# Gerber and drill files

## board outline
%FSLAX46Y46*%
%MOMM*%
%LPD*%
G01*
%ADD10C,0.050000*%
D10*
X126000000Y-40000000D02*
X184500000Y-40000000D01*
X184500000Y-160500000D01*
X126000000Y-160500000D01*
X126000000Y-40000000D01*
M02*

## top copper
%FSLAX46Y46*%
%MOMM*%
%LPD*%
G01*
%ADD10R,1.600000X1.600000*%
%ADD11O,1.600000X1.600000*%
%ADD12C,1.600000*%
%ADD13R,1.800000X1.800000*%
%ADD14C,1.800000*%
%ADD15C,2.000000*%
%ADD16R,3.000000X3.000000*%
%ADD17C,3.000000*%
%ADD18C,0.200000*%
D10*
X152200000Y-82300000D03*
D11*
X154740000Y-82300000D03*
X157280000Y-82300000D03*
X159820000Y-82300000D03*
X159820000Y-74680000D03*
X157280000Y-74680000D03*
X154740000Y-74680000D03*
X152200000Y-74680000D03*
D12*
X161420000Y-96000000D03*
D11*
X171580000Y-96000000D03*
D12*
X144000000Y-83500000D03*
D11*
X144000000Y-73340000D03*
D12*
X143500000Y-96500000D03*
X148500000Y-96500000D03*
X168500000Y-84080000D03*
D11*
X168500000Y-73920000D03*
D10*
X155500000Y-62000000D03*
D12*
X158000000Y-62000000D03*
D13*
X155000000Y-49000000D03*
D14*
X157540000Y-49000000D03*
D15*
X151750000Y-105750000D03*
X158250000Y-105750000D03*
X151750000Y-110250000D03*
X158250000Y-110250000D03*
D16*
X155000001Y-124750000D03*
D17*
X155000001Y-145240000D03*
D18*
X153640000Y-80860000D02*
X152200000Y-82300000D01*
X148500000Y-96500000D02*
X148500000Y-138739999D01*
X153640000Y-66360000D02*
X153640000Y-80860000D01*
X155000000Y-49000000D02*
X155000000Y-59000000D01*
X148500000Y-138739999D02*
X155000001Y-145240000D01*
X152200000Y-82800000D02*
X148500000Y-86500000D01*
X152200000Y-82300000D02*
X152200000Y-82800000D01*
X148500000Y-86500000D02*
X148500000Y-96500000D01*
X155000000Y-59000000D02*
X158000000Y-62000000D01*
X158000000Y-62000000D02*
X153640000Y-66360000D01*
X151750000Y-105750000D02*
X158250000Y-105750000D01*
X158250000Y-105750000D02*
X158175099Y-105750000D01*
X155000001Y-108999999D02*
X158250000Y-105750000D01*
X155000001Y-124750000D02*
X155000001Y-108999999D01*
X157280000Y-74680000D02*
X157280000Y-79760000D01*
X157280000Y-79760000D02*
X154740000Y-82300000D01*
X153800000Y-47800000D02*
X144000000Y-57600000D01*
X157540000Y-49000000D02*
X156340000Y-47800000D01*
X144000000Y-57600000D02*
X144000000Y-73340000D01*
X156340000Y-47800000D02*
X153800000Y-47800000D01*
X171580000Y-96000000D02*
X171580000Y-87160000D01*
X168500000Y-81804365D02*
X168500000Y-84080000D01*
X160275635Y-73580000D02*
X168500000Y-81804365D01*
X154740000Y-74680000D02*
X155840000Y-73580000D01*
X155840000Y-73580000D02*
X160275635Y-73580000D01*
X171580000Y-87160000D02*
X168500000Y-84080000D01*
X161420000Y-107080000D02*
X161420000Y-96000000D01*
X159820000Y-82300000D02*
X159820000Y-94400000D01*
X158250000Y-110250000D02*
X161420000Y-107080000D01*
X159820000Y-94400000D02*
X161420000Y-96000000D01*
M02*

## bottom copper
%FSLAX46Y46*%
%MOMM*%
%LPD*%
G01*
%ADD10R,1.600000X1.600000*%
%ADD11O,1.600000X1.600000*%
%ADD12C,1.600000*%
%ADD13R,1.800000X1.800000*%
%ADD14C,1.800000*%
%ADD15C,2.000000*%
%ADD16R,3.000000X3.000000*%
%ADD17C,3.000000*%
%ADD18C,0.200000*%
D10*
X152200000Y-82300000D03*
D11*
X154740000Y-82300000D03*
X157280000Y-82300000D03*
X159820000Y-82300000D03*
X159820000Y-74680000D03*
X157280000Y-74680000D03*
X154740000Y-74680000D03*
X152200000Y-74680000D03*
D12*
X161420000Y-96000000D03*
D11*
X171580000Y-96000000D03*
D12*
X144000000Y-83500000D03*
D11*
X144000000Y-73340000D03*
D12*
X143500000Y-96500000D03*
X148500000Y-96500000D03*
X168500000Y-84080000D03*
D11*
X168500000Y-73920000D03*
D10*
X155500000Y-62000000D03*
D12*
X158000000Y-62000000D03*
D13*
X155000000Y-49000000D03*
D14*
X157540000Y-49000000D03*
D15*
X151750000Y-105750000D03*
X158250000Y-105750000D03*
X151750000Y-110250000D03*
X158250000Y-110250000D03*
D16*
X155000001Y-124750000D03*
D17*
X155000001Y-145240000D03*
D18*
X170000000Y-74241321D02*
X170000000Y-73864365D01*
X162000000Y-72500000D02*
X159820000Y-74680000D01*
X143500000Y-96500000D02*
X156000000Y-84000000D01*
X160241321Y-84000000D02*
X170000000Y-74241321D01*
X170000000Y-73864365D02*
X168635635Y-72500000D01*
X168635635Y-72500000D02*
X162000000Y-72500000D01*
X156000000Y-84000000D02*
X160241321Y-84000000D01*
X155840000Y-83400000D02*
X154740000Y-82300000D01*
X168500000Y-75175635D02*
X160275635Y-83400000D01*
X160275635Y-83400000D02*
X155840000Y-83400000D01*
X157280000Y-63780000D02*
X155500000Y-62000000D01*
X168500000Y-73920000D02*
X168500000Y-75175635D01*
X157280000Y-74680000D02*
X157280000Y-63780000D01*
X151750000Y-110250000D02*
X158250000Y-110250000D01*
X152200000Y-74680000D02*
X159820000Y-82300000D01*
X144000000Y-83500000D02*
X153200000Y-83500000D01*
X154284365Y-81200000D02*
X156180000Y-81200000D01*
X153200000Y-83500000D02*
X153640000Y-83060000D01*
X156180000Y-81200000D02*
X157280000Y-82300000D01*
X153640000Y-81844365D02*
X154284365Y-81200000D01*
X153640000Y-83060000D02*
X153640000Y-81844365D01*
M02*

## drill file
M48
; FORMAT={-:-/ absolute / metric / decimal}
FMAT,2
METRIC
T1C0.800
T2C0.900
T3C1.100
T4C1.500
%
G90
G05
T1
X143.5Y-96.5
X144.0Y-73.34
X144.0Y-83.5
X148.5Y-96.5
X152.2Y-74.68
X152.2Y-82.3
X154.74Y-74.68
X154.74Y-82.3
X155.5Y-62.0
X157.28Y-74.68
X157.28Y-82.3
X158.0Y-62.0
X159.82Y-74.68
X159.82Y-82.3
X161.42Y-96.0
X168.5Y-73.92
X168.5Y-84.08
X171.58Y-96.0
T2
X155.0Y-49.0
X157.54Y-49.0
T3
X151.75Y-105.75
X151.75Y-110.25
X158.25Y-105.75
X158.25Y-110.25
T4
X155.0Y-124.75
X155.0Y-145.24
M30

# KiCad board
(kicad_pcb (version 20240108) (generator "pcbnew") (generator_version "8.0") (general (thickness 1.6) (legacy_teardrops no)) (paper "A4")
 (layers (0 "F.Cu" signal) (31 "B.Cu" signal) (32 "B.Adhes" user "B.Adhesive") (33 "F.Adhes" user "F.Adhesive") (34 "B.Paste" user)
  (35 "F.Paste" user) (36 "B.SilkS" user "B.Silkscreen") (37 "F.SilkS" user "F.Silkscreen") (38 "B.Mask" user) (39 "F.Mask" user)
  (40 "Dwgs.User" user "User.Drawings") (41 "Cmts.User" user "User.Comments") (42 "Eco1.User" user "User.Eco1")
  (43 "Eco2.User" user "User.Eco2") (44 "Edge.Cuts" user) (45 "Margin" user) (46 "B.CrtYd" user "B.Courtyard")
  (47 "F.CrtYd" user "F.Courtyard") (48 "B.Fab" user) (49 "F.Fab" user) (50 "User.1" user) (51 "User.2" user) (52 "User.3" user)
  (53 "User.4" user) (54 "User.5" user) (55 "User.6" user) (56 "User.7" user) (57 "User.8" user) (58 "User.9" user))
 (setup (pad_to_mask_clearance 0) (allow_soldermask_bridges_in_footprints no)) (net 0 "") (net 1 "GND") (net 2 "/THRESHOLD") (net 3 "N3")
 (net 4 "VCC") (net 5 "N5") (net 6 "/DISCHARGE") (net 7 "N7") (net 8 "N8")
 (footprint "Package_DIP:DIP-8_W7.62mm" (layer "F.Cu") (at 152.2 82.3 90)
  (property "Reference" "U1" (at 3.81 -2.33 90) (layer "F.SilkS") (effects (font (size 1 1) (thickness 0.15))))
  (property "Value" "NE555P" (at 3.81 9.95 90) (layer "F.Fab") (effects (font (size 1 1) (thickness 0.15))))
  (pad "1" thru_hole rect (at 0 0 90) (size 1.6 1.6) (drill 0.8) (layers "*.Cu" "*.Mask") (remove_unused_layers no) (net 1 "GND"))
  (pad "2" thru_hole oval (at 0 2.54 90) (size 1.6 1.6) (drill 0.8) (layers "*.Cu" "*.Mask") (remove_unused_layers no) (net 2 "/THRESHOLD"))
  (pad "3" thru_hole oval (at 0 5.08 90) (size 1.6 1.6) (drill 0.8) (layers "*.Cu" "*.Mask") (remove_unused_layers no) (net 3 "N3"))
  (pad "4" thru_hole oval (at 0 7.62 90) (size 1.6 1.6) (drill 0.8) (layers "*.Cu" "*.Mask") (remove_unused_layers no) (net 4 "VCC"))
  (pad "5" thru_hole oval (at 7.62 7.62 90) (size 1.6 1.6) (drill 0.8) (layers "*.Cu" "*.Mask") (remove_unused_layers no) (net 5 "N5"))
  (pad "6" thru_hole oval (at 7.62 5.08 90) (size 1.6 1.6) (drill 0.8) (layers "*.Cu" "*.Mask") (remove_unused_layers no)
   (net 2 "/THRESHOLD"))
  (pad "7" thru_hole oval (at 7.62 2.54 90) (size 1.6 1.6) (drill 0.8) (layers "*.Cu" "*.Mask") (remove_unused_layers no)
   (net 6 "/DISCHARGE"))
  (pad "8" thru_hole oval (at 7.62 0 90) (size 1.6 1.6) (drill 0.8) (layers "*.Cu" "*.Mask") (remove_unused_layers no) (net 4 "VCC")))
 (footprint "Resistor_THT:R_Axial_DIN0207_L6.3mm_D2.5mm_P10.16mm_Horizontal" (layer "F.Cu") (at 161.42 96)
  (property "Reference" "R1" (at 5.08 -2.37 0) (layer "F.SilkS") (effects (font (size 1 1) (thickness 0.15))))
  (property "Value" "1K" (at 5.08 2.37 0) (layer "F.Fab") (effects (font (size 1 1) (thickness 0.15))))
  (pad "1" thru_hole circle (at 0 0) (size 1.6 1.6) (drill 0.8) (layers "*.Cu" "*.Mask") (remove_unused_layers no) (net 4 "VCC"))
  (pad "2" thru_hole oval (at 10.16 0) (size 1.6 1.6) (drill 0.8) (layers "*.Cu" "*.Mask") (remove_unused_layers no) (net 6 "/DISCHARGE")))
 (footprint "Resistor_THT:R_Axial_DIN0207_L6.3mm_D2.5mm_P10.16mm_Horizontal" (layer "F.Cu") (at 144 83.5 90)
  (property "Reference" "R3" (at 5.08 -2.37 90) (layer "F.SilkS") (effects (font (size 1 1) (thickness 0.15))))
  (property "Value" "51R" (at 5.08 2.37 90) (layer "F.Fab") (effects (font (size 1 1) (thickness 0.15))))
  (pad "1" thru_hole circle (at 0 0 90) (size 1.6 1.6) (drill 0.8) (layers "*.Cu" "*.Mask") (remove_unused_layers no) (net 3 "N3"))
  (pad "2" thru_hole oval (at 10.16 0 90) (size 1.6 1.6) (drill 0.8) (layers "*.Cu" "*.Mask") (remove_unused_layers no) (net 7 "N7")))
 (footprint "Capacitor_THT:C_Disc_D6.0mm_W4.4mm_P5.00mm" (layer "F.Cu") (at 143.5 96.5)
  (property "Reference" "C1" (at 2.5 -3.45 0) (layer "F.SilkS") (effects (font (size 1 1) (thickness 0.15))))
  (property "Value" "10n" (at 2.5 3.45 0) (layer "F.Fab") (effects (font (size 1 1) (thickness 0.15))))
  (pad "1" thru_hole circle (at 0 0) (size 1.6 1.6) (drill 0.8) (layers "*.Cu" "*.Mask") (remove_unused_layers no) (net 5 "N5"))
  (pad "2" thru_hole circle (at 5 0) (size 1.6 1.6) (drill 0.8) (layers "*.Cu" "*.Mask") (remove_unused_layers no) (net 1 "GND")))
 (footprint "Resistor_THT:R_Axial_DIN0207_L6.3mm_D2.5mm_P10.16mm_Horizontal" (layer "F.Cu") (at 168.5 84.08 90)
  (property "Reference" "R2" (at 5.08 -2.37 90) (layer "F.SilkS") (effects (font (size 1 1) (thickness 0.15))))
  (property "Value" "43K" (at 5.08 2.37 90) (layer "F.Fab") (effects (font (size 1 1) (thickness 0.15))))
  (pad "1" thru_hole circle (at 0 0 90) (size 1.6 1.6) (drill 0.8) (layers "*.Cu" "*.Mask") (remove_unused_layers no) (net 6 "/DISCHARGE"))
  (pad "2" thru_hole oval (at 10.16 0 90) (size 1.6 1.6) (drill 0.8) (layers "*.Cu" "*.Mask") (remove_unused_layers no) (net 2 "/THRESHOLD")))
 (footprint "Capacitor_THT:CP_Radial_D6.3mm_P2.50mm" (layer "F.Cu") (at 155.5 62)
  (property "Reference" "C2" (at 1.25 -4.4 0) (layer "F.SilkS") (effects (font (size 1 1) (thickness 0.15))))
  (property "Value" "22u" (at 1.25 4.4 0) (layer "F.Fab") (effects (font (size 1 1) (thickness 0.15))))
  (pad "1" thru_hole rect (at 0 0) (size 1.6 1.6) (drill 0.8) (layers "*.Cu" "*.Mask") (remove_unused_layers no) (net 2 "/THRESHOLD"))
  (pad "2" thru_hole circle (at 2.5 0) (size 1.6 1.6) (drill 0.8) (layers "*.Cu" "*.Mask") (remove_unused_layers no) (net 1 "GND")))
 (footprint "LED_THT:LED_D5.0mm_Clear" (layer "F.Cu") (at 155 49)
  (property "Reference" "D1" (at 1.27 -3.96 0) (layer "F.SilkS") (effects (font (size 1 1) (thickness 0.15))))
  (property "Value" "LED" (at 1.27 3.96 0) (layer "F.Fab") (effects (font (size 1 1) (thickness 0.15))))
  (pad "1" thru_hole rect (at 0 0) (size 1.8 1.8) (drill 0.9) (layers "*.Cu" "*.Mask") (remove_unused_layers no) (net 1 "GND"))
  (pad "2" thru_hole circle (at 2.54 0) (size 1.8 1.8) (drill 0.9) (layers "*.Cu" "*.Mask") (remove_unused_layers no) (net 7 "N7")))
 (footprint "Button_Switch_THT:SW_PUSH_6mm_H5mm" (layer "F.Cu") (at 151.75 105.75)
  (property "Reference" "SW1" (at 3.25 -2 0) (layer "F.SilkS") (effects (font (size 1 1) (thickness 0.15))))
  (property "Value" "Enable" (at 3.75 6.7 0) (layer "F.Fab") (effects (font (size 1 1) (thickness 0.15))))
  (pad "1" thru_hole circle (at 0 0 90) (size 2 2) (drill 1.1) (layers "*.Cu" "*.Mask") (remove_unused_layers no) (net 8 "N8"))
  (pad "1" thru_hole circle (at 6.5 0 90) (size 2 2) (drill 1.1) (layers "*.Cu" "*.Mask") (remove_unused_layers no) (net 8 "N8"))
  (pad "2" thru_hole circle (at 0 4.5 90) (size 2 2) (drill 1.1) (layers "*.Cu" "*.Mask") (remove_unused_layers no) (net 4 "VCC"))
  (pad "2" thru_hole circle (at 6.5 4.5 90) (size 2 2) (drill 1.1) (layers "*.Cu" "*.Mask") (remove_unused_layers no) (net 4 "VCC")))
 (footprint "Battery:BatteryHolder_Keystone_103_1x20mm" (layer "F.Cu") (at 155.000001 124.75 -90)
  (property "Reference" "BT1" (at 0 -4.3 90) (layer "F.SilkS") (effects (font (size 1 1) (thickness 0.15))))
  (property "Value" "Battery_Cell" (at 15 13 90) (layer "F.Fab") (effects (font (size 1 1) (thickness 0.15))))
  (pad "1" thru_hole rect (at 0 0 270) (size 3 3) (drill 1.5) (layers "*.Cu" "*.Mask") (remove_unused_layers no) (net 8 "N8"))
  (pad "2" thru_hole circle (at 20.49 0 270) (size 3 3) (drill 1.5) (layers "*.Cu" "*.Mask") (remove_unused_layers no) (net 1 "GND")))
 (gr_rect (start 126 40) (end 184.5 160.5) (stroke (width 0.05) (type default)) (fill none) (layer "Edge.Cuts"))
 (segment (start 153.64 80.86) (end 152.2 82.3) (width 0.2) (layer "F.Cu") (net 1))
 (segment (start 148.5 96.5) (end 148.5 138.739999) (width 0.2) (layer "F.Cu") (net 1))
 (segment (start 153.64 66.36) (end 153.64 80.86) (width 0.2) (layer "F.Cu") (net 1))
 (segment (start 155 49) (end 155 59) (width 0.2) (layer "F.Cu") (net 1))
 (segment (start 148.5 138.739999) (end 155.000001 145.24) (width 0.2) (layer "F.Cu") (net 1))
 (segment (start 152.2 82.8) (end 148.5 86.5) (width 0.2) (layer "F.Cu") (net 1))
 (segment (start 152.2 82.3) (end 152.2 82.8) (width 0.2) (layer "F.Cu") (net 1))
 (segment (start 148.5 86.5) (end 148.5 96.5) (width 0.2) (layer "F.Cu") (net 1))
 (segment (start 155 59) (end 158 62) (width 0.2) (layer "F.Cu") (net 1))
 (segment (start 158 62) (end 153.64 66.36) (width 0.2) (layer "F.Cu") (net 1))
 (segment (start 151.75 105.75) (end 158.25 105.75) (width 0.2) (layer "F.Cu") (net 8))
 (segment (start 158.25 105.75) (end 158.175099 105.75) (width 0.2) (layer "F.Cu") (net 8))
 (segment (start 155.000001 108.999999) (end 158.25 105.75) (width 0.2) (layer "F.Cu") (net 8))
 (segment (start 155.000001 124.75) (end 155.000001 108.999999) (width 0.2) (layer "F.Cu") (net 8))
 (segment (start 170 74.241321) (end 170 73.864365) (width 0.2) (layer "B.Cu") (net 5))
 (segment (start 162 72.5) (end 159.82 74.68) (width 0.2) (layer "B.Cu") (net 5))
 (segment (start 143.5 96.5) (end 156 84) (width 0.2) (layer "B.Cu") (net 5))
 (segment (start 160.241321 84) (end 170 74.241321) (width 0.2) (layer "B.Cu") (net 5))
 (segment (start 170 73.864365) (end 168.635635 72.5) (width 0.2) (layer "B.Cu") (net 5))
 (segment (start 168.635635 72.5) (end 162 72.5) (width 0.2) (layer "B.Cu") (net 5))
 (segment (start 156 84) (end 160.241321 84) (width 0.2) (layer "B.Cu") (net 5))
 (segment (start 157.28 74.68) (end 157.28 79.76) (width 0.2) (layer "F.Cu") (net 2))
 (segment (start 157.28 79.76) (end 154.74 82.3) (width 0.2) (layer "F.Cu") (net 2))
 (segment (start 155.84 83.4) (end 154.74 82.3) (width 0.2) (layer "B.Cu") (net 2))
 (segment (start 168.5 75.175635) (end 160.275635 83.4) (width 0.2) (layer "B.Cu") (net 2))
 (segment (start 160.275635 83.4) (end 155.84 83.4) (width 0.2) (layer "B.Cu") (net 2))
 (segment (start 157.28 63.78) (end 155.5 62) (width 0.2) (layer "B.Cu") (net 2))
 (segment (start 168.5 73.92) (end 168.5 75.175635) (width 0.2) (layer "B.Cu") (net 2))
 (segment (start 157.28 74.68) (end 157.28 63.78) (width 0.2) (layer "B.Cu") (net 2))
 (segment (start 153.8 47.8) (end 144 57.6) (width 0.2) (layer "F.Cu") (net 7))
 (segment (start 157.54 49) (end 156.34 47.8) (width 0.2) (layer "F.Cu") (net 7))
 (segment (start 144 57.6) (end 144 73.34) (width 0.2) (layer "F.Cu") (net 7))
 (segment (start 156.34 47.8) (end 153.8 47.8) (width 0.2) (layer "F.Cu") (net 7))
 (segment (start 171.58 96) (end 171.58 87.16) (width 0.2) (layer "F.Cu") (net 6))
 (segment (start 168.5 81.804365) (end 168.5 84.08) (width 0.2) (layer "F.Cu") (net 6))
 (segment (start 160.275635 73.58) (end 168.5 81.804365) (width 0.2) (layer "F.Cu") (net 6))
 (segment (start 154.74 74.68) (end 155.84 73.58) (width 0.2) (layer "F.Cu") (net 6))
 (segment (start 155.84 73.58) (end 160.275635 73.58) (width 0.2) (layer "F.Cu") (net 6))
 (segment (start 171.58 87.16) (end 168.5 84.08) (width 0.2) (layer "F.Cu") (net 6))
 (segment (start 161.42 107.08) (end 161.42 96) (width 0.2) (layer "F.Cu") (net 4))
 (segment (start 159.82 82.3) (end 159.82 94.4) (width 0.2) (layer "F.Cu") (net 4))
 (segment (start 158.25 110.25) (end 161.42 107.08) (width 0.2) (layer "F.Cu") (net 4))
 (segment (start 159.82 94.4) (end 161.42 96) (width 0.2) (layer "F.Cu") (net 4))
 (segment (start 151.75 110.25) (end 158.25 110.25) (width 0.2) (layer "B.Cu") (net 4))
 (segment (start 152.2 74.68) (end 159.82 82.3) (width 0.2) (layer "B.Cu") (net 4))
 (segment (start 144 83.5) (end 153.2 83.5) (width 0.2) (layer "B.Cu") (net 3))
 (segment (start 154.284365 81.2) (end 156.18 81.2) (width 0.2) (layer "B.Cu") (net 3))
 (segment (start 153.2 83.5) (end 153.64 83.06) (width 0.2) (layer "B.Cu") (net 3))
 (segment (start 156.18 81.2) (end 157.28 82.3) (width 0.2) (layer "B.Cu") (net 3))
 (segment (start 153.64 81.844365) (end 154.284365 81.2) (width 0.2) (layer "B.Cu") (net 3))
 (segment (start 153.64 83.06) (end 153.64 81.844365) (width 0.2) (layer "B.Cu") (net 3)))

